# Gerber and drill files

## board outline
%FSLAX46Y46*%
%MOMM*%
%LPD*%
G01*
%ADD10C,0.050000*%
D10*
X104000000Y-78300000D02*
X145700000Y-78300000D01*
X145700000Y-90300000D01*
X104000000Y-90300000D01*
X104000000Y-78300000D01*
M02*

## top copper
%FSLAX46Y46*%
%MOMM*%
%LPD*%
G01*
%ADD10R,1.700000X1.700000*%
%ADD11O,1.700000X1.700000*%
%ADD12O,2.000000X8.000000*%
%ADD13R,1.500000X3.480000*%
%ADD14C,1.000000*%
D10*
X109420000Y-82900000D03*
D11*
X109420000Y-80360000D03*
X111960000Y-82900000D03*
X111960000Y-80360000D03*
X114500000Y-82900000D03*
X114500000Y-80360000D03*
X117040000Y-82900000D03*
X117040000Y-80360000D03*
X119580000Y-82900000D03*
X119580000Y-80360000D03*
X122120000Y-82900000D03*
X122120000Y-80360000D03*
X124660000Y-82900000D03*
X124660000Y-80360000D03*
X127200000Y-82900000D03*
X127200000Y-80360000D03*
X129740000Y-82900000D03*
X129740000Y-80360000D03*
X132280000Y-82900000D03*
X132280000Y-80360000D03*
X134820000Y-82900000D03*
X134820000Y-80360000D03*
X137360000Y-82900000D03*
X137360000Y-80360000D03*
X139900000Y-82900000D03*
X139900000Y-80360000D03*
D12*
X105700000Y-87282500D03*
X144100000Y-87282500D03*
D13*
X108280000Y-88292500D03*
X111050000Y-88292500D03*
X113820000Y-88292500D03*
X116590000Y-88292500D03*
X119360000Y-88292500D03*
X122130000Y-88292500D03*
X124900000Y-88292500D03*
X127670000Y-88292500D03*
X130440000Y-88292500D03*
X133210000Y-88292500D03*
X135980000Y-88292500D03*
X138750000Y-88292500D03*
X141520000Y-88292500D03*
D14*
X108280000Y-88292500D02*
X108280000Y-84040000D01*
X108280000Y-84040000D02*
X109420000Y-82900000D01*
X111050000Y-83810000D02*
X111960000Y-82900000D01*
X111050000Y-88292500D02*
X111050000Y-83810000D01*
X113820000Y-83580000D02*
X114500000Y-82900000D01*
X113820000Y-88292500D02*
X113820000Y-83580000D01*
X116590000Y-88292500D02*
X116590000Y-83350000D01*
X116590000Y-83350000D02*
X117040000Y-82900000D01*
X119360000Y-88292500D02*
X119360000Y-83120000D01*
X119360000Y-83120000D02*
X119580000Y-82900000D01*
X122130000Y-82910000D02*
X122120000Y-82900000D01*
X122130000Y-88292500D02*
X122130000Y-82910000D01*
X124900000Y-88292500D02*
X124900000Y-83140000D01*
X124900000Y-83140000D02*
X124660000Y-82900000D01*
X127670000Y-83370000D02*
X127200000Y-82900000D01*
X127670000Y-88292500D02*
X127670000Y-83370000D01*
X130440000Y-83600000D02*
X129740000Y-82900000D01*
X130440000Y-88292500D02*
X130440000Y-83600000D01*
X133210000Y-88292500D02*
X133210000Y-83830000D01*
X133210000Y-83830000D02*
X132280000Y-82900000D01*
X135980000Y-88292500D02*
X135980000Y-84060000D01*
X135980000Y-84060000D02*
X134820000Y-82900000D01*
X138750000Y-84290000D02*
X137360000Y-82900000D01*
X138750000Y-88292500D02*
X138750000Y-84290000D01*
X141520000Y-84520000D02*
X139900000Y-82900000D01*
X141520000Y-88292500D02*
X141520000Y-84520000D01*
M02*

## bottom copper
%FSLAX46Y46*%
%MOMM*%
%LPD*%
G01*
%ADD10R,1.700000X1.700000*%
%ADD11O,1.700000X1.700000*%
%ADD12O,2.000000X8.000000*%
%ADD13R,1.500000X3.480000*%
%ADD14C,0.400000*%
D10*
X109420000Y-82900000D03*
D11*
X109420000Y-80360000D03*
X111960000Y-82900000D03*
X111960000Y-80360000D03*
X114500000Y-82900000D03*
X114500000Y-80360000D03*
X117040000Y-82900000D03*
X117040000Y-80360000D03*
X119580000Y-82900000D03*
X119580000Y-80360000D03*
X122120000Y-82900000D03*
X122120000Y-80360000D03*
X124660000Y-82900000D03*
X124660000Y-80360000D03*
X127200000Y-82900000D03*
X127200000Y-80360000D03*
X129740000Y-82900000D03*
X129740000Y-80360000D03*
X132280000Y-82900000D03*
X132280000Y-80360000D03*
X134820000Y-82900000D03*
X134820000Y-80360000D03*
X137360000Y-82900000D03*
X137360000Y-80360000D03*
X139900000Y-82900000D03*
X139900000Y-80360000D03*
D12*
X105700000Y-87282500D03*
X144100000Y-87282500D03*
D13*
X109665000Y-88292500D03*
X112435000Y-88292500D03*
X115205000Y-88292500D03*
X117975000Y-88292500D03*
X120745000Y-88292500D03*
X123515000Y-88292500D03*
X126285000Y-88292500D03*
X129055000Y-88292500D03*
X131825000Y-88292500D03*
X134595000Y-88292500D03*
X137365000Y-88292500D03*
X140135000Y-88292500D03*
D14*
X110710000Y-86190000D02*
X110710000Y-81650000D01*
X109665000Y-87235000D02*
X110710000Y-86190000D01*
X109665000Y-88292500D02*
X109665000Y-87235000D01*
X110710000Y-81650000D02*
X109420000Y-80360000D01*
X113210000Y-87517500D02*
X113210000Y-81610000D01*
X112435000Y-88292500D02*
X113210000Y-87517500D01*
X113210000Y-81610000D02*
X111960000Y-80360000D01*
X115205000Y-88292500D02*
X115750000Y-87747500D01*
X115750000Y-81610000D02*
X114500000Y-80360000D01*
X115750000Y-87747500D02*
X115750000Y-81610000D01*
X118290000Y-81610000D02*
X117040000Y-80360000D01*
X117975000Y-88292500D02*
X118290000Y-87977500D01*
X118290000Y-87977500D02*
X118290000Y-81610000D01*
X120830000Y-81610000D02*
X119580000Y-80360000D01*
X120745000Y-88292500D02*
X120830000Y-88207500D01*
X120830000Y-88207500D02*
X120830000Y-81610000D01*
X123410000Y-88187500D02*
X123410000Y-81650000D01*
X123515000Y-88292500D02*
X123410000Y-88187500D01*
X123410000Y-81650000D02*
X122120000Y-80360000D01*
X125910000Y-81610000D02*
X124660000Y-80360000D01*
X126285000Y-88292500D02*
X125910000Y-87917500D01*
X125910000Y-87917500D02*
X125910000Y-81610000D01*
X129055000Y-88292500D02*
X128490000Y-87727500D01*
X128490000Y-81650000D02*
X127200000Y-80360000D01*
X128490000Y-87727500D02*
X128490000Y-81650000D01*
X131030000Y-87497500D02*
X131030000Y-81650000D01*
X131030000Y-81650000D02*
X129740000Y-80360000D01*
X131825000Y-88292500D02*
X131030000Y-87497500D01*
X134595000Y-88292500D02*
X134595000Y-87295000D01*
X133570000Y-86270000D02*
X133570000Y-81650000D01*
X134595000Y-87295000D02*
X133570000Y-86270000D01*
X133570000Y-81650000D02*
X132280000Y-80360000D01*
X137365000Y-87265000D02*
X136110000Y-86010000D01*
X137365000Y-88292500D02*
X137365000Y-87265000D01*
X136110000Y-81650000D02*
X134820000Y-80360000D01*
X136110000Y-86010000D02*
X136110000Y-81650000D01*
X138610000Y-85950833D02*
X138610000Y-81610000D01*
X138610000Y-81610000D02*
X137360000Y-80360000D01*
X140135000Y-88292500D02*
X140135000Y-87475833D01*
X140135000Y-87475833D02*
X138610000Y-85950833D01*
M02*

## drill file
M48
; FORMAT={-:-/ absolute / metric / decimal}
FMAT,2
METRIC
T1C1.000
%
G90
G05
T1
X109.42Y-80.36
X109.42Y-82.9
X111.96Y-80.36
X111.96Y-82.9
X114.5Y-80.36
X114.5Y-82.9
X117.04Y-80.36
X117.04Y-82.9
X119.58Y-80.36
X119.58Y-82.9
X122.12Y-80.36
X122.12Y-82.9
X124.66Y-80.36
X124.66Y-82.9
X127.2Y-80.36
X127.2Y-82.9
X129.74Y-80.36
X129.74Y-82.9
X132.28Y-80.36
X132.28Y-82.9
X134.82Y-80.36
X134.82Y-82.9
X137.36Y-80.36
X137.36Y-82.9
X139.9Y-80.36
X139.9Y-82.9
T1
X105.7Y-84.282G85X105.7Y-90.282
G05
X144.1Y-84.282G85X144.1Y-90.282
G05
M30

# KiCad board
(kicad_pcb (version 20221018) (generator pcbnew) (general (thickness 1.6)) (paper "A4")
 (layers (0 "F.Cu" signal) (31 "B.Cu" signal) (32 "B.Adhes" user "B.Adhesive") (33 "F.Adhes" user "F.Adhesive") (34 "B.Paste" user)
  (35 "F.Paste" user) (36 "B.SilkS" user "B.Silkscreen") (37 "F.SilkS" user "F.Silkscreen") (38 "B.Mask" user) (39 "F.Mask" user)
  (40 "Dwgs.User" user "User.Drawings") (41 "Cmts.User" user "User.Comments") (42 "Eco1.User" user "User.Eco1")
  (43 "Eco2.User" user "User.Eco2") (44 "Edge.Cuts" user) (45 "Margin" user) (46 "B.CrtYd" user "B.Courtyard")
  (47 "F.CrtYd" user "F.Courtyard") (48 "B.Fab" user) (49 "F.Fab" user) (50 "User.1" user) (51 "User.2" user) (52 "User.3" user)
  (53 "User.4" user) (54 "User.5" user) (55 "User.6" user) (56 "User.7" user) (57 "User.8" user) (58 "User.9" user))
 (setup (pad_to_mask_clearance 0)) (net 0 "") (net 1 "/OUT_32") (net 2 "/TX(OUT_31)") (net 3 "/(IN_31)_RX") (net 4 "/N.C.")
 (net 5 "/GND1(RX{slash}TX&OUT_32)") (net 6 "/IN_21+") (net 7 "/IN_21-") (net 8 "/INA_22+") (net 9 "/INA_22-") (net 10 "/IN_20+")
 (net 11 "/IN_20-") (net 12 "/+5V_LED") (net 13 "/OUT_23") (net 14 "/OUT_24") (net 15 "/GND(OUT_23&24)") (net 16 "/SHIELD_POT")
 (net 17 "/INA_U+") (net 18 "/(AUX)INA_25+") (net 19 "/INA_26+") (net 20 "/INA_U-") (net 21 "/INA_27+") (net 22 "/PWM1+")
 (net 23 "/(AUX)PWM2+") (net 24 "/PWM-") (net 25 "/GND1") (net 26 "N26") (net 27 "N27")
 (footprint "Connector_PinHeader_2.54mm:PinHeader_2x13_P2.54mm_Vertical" (layer "F.Cu") (at 109.42 82.9 90)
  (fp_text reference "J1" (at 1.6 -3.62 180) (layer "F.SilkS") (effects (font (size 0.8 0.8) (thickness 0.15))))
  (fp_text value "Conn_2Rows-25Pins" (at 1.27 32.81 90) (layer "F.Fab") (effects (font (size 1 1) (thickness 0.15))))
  (pad "1" thru_hole rect (at 0 0 90) (size 1.7 1.7) (drill 1) (layers "*.Cu" "*.Mask") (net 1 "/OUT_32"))
  (pad "2" thru_hole oval (at 2.54 0 90) (size 1.7 1.7) (drill 1) (layers "*.Cu" "*.Mask") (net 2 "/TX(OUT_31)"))
  (pad "3" thru_hole oval (at 0 2.54 90) (size 1.7 1.7) (drill 1) (layers "*.Cu" "*.Mask") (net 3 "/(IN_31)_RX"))
  (pad "4" thru_hole oval (at 2.54 2.54 90) (size 1.7 1.7) (drill 1) (layers "*.Cu" "*.Mask") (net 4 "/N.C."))
  (pad "5" thru_hole oval (at 0 5.08 90) (size 1.7 1.7) (drill 1) (layers "*.Cu" "*.Mask") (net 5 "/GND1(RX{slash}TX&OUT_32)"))
  (pad "6" thru_hole oval (at 2.54 5.08 90) (size 1.7 1.7) (drill 1) (layers "*.Cu" "*.Mask") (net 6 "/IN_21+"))
  (pad "7" thru_hole oval (at 0 7.62 90) (size 1.7 1.7) (drill 1) (layers "*.Cu" "*.Mask") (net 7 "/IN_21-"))
  (pad "8" thru_hole oval (at 2.54 7.62 90) (size 1.7 1.7) (drill 1) (layers "*.Cu" "*.Mask") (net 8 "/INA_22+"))
  (pad "9" thru_hole oval (at 0 10.16 90) (size 1.7 1.7) (drill 1) (layers "*.Cu" "*.Mask") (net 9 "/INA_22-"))
  (pad "10" thru_hole oval (at 2.54 10.16 90) (size 1.7 1.7) (drill 1) (layers "*.Cu" "*.Mask") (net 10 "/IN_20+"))
  (pad "11" thru_hole oval (at 0 12.7 90) (size 1.7 1.7) (drill 1) (layers "*.Cu" "*.Mask") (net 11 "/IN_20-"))
  (pad "12" thru_hole oval (at 2.54 12.7 90) (size 1.7 1.7) (drill 1) (layers "*.Cu" "*.Mask") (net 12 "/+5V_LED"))
  (pad "13" thru_hole oval (at 0 15.24 90) (size 1.7 1.7) (drill 1) (layers "*.Cu" "*.Mask") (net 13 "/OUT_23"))
  (pad "14" thru_hole oval (at 2.54 15.24 90) (size 1.7 1.7) (drill 1) (layers "*.Cu" "*.Mask") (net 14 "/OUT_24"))
  (pad "15" thru_hole oval (at 0 17.78 90) (size 1.7 1.7) (drill 1) (layers "*.Cu" "*.Mask") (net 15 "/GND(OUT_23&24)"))
  (pad "16" thru_hole oval (at 2.54 17.78 90) (size 1.7 1.7) (drill 1) (layers "*.Cu" "*.Mask") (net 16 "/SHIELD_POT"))
  (pad "17" thru_hole oval (at 0 20.32 90) (size 1.7 1.7) (drill 1) (layers "*.Cu" "*.Mask") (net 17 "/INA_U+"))
  (pad "18" thru_hole oval (at 2.54 20.32 90) (size 1.7 1.7) (drill 1) (layers "*.Cu" "*.Mask") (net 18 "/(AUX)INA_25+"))
  (pad "19" thru_hole oval (at 0 22.86 90) (size 1.7 1.7) (drill 1) (layers "*.Cu" "*.Mask") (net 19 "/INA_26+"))
  (pad "20" thru_hole oval (at 2.54 22.86 90) (size 1.7 1.7) (drill 1) (layers "*.Cu" "*.Mask") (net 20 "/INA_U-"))
  (pad "21" thru_hole oval (at 0 25.4 90) (size 1.7 1.7) (drill 1) (layers "*.Cu" "*.Mask") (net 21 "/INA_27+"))
  (pad "22" thru_hole oval (at 2.54 25.4 90) (size 1.7 1.7) (drill 1) (layers "*.Cu" "*.Mask") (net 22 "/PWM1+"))
  (pad "23" thru_hole oval (at 0 27.94 90) (size 1.7 1.7) (drill 1) (layers "*.Cu" "*.Mask") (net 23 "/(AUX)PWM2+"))
  (pad "24" thru_hole oval (at 2.54 27.94 90) (size 1.7 1.7) (drill 1) (layers "*.Cu" "*.Mask") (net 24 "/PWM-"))
  (pad "25" thru_hole oval (at 0 30.48 90) (size 1.7 1.7) (drill 1) (layers "*.Cu" "*.Mask") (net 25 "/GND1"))
  (pad "26" thru_hole oval (at 2.54 30.48 90) (size 1.7 1.7) (drill 1) (layers "*.Cu" "*.Mask") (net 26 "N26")))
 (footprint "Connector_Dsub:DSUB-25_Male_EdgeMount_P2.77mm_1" (layer "F.Cu") (at 124.9 88.2925)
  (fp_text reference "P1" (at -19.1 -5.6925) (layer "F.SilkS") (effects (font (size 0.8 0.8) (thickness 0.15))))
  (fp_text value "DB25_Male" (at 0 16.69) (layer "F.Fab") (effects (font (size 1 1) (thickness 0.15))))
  (pad "0" thru_hole oval (at -19.2 -1.01) (size 2 8) (drill oval 1 7) (layers "*.Cu" "*.Mask") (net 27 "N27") (thermal_bridge_angle 45))
  (pad "0" thru_hole oval (at 19.2 -1.01) (size 2 8) (drill oval 1 7) (layers "*.Cu" "*.Mask") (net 27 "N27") (thermal_bridge_angle 45))
  (pad "1" smd rect (at -16.62 0) (size 1.5 3.48) (layers "F.Cu" "F.Paste" "F.Mask") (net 1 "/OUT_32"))
  (pad "2" smd rect (at -13.85 0) (size 1.5 3.48) (layers "F.Cu" "F.Paste" "F.Mask") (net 3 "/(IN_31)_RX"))
  (pad "3" smd rect (at -11.08 0) (size 1.5 3.48) (layers "F.Cu" "F.Paste" "F.Mask") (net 5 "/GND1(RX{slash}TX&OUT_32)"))
  (pad "4" smd rect (at -8.31 0) (size 1.5 3.48) (layers "F.Cu" "F.Paste" "F.Mask") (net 7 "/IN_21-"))
  (pad "5" smd rect (at -5.54 0) (size 1.5 3.48) (layers "F.Cu" "F.Paste" "F.Mask") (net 9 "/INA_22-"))
  (pad "6" smd rect (at -2.77 0) (size 1.5 3.48) (layers "F.Cu" "F.Paste" "F.Mask") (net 11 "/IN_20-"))
  (pad "7" smd rect (at 0 0) (size 1.5 3.48) (layers "F.Cu" "F.Paste" "F.Mask") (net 13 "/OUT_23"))
  (pad "8" smd rect (at 2.77 0) (size 1.5 3.48) (layers "F.Cu" "F.Paste" "F.Mask") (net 15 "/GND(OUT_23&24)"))
  (pad "9" smd rect (at 5.54 0) (size 1.5 3.48) (layers "F.Cu" "F.Paste" "F.Mask") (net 17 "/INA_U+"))
  (pad "10" smd rect (at 8.31 0) (size 1.5 3.48) (layers "F.Cu" "F.Paste" "F.Mask") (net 19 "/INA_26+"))
  (pad "11" smd rect (at 11.08 0) (size 1.5 3.48) (layers "F.Cu" "F.Paste" "F.Mask") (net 21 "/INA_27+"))
  (pad "12" smd rect (at 13.85 0) (size 1.5 3.48) (layers "F.Cu" "F.Paste" "F.Mask") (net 23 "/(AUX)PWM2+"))
  (pad "13" smd rect (at 16.62 0) (size 1.5 3.48) (layers "F.Cu" "F.Paste" "F.Mask") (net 25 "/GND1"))
  (pad "14" smd rect (at -15.235 0) (size 1.5 3.48) (layers "B.Cu" "B.Paste" "B.Mask") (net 2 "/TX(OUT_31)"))
  (pad "15" smd rect (at -12.465 0) (size 1.5 3.48) (layers "B.Cu" "B.Paste" "B.Mask") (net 4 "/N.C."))
  (pad "16" smd rect (at -9.695 0) (size 1.5 3.48) (layers "B.Cu" "B.Paste" "B.Mask") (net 6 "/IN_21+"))
  (pad "17" smd rect (at -6.925 0) (size 1.5 3.48) (layers "B.Cu" "B.Paste" "B.Mask") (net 8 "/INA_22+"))
  (pad "18" smd rect (at -4.155 0) (size 1.5 3.48) (layers "B.Cu" "B.Paste" "B.Mask") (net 10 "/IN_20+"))
  (pad "19" smd rect (at -1.385 0) (size 1.5 3.48) (layers "B.Cu" "B.Paste" "B.Mask") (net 12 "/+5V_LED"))
  (pad "20" smd rect (at 1.385 0) (size 1.5 3.48) (layers "B.Cu" "B.Paste" "B.Mask") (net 14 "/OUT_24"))
  (pad "21" smd rect (at 4.155 0) (size 1.5 3.48) (layers "B.Cu" "B.Paste" "B.Mask") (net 16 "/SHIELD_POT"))
  (pad "22" smd rect (at 6.925 0) (size 1.5 3.48) (layers "B.Cu" "B.Paste" "B.Mask") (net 18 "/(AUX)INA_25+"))
  (pad "23" smd rect (at 9.695 0) (size 1.5 3.48) (layers "B.Cu" "B.Paste" "B.Mask") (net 20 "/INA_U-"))
  (pad "24" smd rect (at 12.465 0) (size 1.5 3.48) (layers "B.Cu" "B.Paste" "B.Mask") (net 22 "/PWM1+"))
  (pad "25" smd rect (at 15.235 0) (size 1.5 3.48) (layers "B.Cu" "B.Paste" "B.Mask") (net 24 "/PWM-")))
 (gr_rect (start 104 78.3) (end 145.7 90.3) (stroke (width 0.05) (type default)) (fill none) (layer "Edge.Cuts"))
 (segment (start 108.28 88.2925) (end 108.28 84.04) (width 1) (layer "F.Cu") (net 1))
 (segment (start 108.28 84.04) (end 109.42 82.9) (width 1) (layer "F.Cu") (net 1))
 (segment (start 110.71 86.19) (end 110.71 81.65) (width 0.4) (layer "B.Cu") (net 2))
 (segment (start 109.665 87.235) (end 110.71 86.19) (width 0.4) (layer "B.Cu") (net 2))
 (segment (start 109.665 88.2925) (end 109.665 87.235) (width 0.4) (layer "B.Cu") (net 2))
 (segment (start 110.71 81.65) (end 109.42 80.36) (width 0.4) (layer "B.Cu") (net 2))
 (segment (start 111.05 83.81) (end 111.96 82.9) (width 1) (layer "F.Cu") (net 3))
 (segment (start 111.05 88.2925) (end 111.05 83.81) (width 1) (layer "F.Cu") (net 3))
 (segment (start 113.21 87.5175) (end 113.21 81.61) (width 0.4) (layer "B.Cu") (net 4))
 (segment (start 112.435 88.2925) (end 113.21 87.5175) (width 0.4) (layer "B.Cu") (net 4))
 (segment (start 113.21 81.61) (end 111.96 80.36) (width 0.4) (layer "B.Cu") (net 4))
 (segment (start 113.82 83.58) (end 114.5 82.9) (width 1) (layer "F.Cu") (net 5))
 (segment (start 113.82 88.2925) (end 113.82 83.58) (width 1) (layer "F.Cu") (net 5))
 (segment (start 115.205 88.2925) (end 115.75 87.7475) (width 0.4) (layer "B.Cu") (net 6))
 (segment (start 115.75 81.61) (end 114.5 80.36) (width 0.4) (layer "B.Cu") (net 6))
 (segment (start 115.75 87.7475) (end 115.75 81.61) (width 0.4) (layer "B.Cu") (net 6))
 (segment (start 116.59 88.2925) (end 116.59 83.35) (width 1) (layer "F.Cu") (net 7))
 (segment (start 116.59 83.35) (end 117.04 82.9) (width 1) (layer "F.Cu") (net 7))
 (segment (start 118.29 81.61) (end 117.04 80.36) (width 0.4) (layer "B.Cu") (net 8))
 (segment (start 117.975 88.2925) (end 118.29 87.9775) (width 0.4) (layer "B.Cu") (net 8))
 (segment (start 118.29 87.9775) (end 118.29 81.61) (width 0.4) (layer "B.Cu") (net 8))
 (segment (start 119.36 88.2925) (end 119.36 83.12) (width 1) (layer "F.Cu") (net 9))
 (segment (start 119.36 83.12) (end 119.58 82.9) (width 1) (layer "F.Cu") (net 9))
 (segment (start 120.83 81.61) (end 119.58 80.36) (width 0.4) (layer "B.Cu") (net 10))
 (segment (start 120.745 88.2925) (end 120.83 88.2075) (width 0.4) (layer "B.Cu") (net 10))
 (segment (start 120.83 88.2075) (end 120.83 81.61) (width 0.4) (layer "B.Cu") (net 10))
 (segment (start 122.13 82.91) (end 122.12 82.9) (width 1) (layer "F.Cu") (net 11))
 (segment (start 122.13 88.2925) (end 122.13 82.91) (width 1) (layer "F.Cu") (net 11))
 (segment (start 123.41 88.1875) (end 123.41 81.65) (width 0.4) (layer "B.Cu") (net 12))
 (segment (start 123.515 88.2925) (end 123.41 88.1875) (width 0.4) (layer "B.Cu") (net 12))
 (segment (start 123.41 81.65) (end 122.12 80.36) (width 0.4) (layer "B.Cu") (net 12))
 (segment (start 124.9 88.2925) (end 124.9 83.14) (width 1) (layer "F.Cu") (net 13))
 (segment (start 124.9 83.14) (end 124.66 82.9) (width 1) (layer "F.Cu") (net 13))
 (segment (start 125.91 81.61) (end 124.66 80.36) (width 0.4) (layer "B.Cu") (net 14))
 (segment (start 126.285 88.2925) (end 125.91 87.9175) (width 0.4) (layer "B.Cu") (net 14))
 (segment (start 125.91 87.9175) (end 125.91 81.61) (width 0.4) (layer "B.Cu") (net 14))
 (segment (start 127.67 83.37) (end 127.2 82.9) (width 1) (layer "F.Cu") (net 15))
 (segment (start 127.67 88.2925) (end 127.67 83.37) (width 1) (layer "F.Cu") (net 15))
 (segment (start 129.055 88.2925) (end 128.49 87.7275) (width 0.4) (layer "B.Cu") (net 16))
 (segment (start 128.49 81.65) (end 127.2 80.36) (width 0.4) (layer "B.Cu") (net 16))
 (segment (start 128.49 87.7275) (end 128.49 81.65) (width 0.4) (layer "B.Cu") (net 16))
 (segment (start 130.44 83.6) (end 129.74 82.9) (width 1) (layer "F.Cu") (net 17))
 (segment (start 130.44 88.2925) (end 130.44 83.6) (width 1) (layer "F.Cu") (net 17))
 (segment (start 131.03 87.4975) (end 131.03 81.65) (width 0.4) (layer "B.Cu") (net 18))
 (segment (start 131.03 81.65) (end 129.74 80.36) (width 0.4) (layer "B.Cu") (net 18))
 (segment (start 131.825 88.2925) (end 131.03 87.4975) (width 0.4) (layer "B.Cu") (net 18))
 (segment (start 133.21 88.2925) (end 133.21 83.83) (width 1) (layer "F.Cu") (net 19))
 (segment (start 133.21 83.83) (end 132.28 82.9) (width 1) (layer "F.Cu") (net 19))
 (segment (start 134.595 88.2925) (end 134.595 87.295) (width 0.4) (layer "B.Cu") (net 20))
 (segment (start 133.57 86.27) (end 133.57 81.65) (width 0.4) (layer "B.Cu") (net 20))
 (segment (start 134.595 87.295) (end 133.57 86.27) (width 0.4) (layer "B.Cu") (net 20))
 (segment (start 133.57 81.65) (end 132.28 80.36) (width 0.4) (layer "B.Cu") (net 20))
 (segment (start 135.98 88.2925) (end 135.98 84.06) (width 1) (layer "F.Cu") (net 21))
 (segment (start 135.98 84.06) (end 134.82 82.9) (width 1) (layer "F.Cu") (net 21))
 (segment (start 137.365 87.265) (end 136.11 86.01) (width 0.4) (layer "B.Cu") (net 22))
 (segment (start 137.365 88.2925) (end 137.365 87.265) (width 0.4) (layer "B.Cu") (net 22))
 (segment (start 136.11 81.65) (end 134.82 80.36) (width 0.4) (layer "B.Cu") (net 22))
 (segment (start 136.11 86.01) (end 136.11 81.65) (width 0.4) (layer "B.Cu") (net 22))
 (segment (start 138.75 84.29) (end 137.36 82.9) (width 1) (layer "F.Cu") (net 23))
 (segment (start 138.75 88.2925) (end 138.75 84.29) (width 1) (layer "F.Cu") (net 23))
 (segment (start 138.61 85.950833) (end 138.61 81.61) (width 0.4) (layer "B.Cu") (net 24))
 (segment (start 138.61 81.61) (end 137.36 80.36) (width 0.4) (layer "B.Cu") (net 24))
 (segment (start 140.135 88.2925) (end 140.135 87.475833) (width 0.4) (layer "B.Cu") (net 24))
 (segment (start 140.135 87.475833) (end 138.61 85.950833) (width 0.4) (layer "B.Cu") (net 24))
 (segment (start 141.52 84.52) (end 139.9 82.9) (width 1) (layer "F.Cu") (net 25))
 (segment (start 141.52 88.2925) (end 141.52 84.52) (width 1) (layer "F.Cu") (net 25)))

